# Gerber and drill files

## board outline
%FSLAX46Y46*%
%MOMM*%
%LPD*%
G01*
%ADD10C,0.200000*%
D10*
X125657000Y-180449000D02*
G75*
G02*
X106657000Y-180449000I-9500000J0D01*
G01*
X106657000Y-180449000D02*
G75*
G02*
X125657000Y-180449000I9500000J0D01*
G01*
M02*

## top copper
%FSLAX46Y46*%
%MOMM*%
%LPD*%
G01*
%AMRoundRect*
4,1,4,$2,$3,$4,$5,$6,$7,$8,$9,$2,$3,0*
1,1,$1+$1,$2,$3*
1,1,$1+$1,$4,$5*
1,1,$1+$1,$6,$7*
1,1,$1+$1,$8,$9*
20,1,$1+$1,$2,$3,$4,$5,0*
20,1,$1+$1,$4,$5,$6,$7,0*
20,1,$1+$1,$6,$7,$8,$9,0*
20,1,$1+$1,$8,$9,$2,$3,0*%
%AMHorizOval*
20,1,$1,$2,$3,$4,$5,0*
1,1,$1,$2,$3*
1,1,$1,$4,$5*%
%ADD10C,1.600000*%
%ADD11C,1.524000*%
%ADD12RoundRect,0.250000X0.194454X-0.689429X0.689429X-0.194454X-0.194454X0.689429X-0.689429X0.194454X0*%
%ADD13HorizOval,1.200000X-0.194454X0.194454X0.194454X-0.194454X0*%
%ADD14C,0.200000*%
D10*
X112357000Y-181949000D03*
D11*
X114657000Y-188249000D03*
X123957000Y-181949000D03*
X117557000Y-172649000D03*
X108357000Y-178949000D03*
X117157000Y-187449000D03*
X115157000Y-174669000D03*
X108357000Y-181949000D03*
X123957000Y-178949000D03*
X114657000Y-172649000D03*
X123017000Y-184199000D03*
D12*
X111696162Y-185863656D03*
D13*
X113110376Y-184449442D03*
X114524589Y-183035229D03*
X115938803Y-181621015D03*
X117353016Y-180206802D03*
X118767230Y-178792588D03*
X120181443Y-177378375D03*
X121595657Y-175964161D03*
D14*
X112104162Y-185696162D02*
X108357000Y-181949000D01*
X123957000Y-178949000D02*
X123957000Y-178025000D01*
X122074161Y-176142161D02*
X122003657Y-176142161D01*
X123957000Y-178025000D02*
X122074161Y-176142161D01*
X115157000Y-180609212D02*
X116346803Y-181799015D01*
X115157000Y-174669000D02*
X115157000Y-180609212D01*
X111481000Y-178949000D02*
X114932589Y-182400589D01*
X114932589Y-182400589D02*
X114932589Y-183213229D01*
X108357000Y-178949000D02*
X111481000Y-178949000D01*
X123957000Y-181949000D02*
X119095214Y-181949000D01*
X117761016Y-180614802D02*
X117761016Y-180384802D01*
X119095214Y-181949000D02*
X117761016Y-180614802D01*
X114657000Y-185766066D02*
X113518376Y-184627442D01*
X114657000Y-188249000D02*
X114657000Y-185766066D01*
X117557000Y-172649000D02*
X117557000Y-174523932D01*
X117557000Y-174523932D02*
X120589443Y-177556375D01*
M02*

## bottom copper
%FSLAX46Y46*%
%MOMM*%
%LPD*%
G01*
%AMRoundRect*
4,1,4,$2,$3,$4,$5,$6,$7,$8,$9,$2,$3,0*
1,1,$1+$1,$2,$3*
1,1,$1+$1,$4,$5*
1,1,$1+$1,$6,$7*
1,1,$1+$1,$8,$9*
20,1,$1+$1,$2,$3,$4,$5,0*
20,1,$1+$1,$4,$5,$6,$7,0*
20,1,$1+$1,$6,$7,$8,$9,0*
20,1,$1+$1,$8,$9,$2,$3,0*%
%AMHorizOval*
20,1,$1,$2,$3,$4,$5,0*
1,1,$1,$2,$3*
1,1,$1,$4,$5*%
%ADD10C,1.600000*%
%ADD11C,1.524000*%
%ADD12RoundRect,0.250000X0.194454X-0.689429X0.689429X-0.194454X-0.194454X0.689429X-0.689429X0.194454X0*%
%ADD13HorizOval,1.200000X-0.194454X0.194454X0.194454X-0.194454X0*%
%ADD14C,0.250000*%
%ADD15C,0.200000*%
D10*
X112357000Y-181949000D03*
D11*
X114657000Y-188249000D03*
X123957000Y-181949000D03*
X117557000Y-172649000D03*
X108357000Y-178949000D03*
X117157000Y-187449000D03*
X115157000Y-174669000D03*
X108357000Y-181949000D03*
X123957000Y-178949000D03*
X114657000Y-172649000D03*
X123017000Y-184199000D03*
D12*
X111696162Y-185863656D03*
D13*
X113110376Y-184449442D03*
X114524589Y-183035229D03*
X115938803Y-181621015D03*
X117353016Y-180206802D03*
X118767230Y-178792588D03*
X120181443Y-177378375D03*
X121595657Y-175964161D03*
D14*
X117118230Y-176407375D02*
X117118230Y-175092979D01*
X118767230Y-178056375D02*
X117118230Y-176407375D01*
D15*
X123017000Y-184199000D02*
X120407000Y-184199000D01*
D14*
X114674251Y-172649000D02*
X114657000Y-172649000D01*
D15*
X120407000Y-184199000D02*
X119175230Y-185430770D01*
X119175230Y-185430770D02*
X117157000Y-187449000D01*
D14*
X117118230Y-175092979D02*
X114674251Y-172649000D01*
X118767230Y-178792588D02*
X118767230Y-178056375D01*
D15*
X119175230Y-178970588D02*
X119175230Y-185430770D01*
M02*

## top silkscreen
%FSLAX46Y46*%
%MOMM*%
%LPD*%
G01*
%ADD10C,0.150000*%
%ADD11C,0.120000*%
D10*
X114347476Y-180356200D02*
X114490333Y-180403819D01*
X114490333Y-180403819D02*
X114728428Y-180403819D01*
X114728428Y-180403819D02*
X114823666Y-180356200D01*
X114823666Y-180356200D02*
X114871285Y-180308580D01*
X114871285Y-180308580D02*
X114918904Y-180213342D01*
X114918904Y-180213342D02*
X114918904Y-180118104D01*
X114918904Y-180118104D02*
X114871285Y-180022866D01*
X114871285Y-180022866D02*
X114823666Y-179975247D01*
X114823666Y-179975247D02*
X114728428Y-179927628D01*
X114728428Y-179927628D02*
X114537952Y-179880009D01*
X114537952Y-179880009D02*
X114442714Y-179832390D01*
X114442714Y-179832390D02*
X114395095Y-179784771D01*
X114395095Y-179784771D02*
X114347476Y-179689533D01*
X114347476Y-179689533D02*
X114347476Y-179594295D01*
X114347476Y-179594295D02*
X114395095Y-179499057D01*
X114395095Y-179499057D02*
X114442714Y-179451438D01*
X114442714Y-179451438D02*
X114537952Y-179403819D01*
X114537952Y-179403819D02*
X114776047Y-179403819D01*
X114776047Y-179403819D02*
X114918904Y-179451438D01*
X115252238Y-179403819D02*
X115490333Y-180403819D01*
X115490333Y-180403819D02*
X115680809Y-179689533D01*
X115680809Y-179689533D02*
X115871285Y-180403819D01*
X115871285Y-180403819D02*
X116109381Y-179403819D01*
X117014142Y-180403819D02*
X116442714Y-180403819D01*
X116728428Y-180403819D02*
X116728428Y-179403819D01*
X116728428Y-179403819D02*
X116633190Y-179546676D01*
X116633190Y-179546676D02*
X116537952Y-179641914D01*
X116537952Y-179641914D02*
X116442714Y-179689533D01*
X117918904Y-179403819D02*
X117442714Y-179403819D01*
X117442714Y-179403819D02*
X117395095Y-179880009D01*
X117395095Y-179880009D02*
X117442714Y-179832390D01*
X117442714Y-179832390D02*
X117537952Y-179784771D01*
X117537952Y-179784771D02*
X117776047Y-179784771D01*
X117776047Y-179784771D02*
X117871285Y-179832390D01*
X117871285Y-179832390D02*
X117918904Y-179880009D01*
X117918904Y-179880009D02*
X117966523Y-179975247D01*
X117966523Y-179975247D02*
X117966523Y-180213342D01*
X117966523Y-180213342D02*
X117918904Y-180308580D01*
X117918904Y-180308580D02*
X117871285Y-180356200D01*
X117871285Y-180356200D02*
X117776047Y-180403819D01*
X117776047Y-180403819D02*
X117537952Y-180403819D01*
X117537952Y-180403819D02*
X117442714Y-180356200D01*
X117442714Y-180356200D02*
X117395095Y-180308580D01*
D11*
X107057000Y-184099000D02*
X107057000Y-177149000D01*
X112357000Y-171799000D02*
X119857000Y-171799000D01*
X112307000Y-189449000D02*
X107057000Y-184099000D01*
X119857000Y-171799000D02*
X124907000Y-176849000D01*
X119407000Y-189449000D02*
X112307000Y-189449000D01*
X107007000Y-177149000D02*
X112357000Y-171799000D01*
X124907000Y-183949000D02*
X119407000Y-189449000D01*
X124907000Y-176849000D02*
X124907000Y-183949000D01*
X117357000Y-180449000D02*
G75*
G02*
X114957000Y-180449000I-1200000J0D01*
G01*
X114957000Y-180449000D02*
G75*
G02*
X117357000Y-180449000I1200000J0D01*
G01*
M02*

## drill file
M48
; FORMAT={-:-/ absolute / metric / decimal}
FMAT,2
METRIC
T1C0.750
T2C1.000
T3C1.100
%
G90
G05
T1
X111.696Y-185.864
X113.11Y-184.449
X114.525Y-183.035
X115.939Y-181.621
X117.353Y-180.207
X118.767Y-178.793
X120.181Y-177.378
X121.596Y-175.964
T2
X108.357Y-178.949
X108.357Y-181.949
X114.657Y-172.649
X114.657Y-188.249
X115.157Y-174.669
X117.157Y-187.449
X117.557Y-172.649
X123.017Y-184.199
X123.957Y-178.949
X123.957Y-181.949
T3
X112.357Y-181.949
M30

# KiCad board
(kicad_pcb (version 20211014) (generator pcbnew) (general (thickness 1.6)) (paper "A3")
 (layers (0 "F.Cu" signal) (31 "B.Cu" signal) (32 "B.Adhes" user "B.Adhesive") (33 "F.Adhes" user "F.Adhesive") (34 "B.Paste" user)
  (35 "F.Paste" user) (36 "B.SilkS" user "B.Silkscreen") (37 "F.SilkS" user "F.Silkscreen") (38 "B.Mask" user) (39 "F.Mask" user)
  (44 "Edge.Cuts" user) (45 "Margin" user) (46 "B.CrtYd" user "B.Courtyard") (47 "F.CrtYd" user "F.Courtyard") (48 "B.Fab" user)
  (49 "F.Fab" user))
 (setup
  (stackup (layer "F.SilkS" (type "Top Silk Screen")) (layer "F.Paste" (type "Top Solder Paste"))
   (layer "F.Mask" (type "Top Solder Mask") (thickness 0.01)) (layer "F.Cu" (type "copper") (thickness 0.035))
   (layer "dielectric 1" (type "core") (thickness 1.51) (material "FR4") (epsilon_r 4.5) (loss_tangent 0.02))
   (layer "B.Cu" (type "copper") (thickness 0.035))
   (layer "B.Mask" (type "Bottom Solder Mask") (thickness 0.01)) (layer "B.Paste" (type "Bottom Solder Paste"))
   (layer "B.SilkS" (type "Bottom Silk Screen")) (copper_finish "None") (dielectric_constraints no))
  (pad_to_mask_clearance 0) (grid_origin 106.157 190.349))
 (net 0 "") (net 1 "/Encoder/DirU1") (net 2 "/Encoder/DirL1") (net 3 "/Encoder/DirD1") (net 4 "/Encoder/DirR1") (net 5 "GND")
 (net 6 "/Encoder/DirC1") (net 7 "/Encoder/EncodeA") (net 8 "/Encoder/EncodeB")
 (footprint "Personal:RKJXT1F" (layer "F.Cu") (at 116.157 180.449)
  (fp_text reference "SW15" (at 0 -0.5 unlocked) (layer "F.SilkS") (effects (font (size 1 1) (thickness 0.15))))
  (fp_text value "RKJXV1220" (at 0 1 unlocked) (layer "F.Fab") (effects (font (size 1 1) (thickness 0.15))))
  (fp_line (start -9.1 3.65) (end -9.1 -3.3) (layer "F.SilkS") (width 0.12))
  (fp_line (start -3.8 -8.65) (end 3.7 -8.65) (layer "F.SilkS") (width 0.12))
  (fp_line (start -3.85 9) (end -9.1 3.65) (layer "F.SilkS") (width 0.12))
  (fp_line (start 3.7 -8.65) (end 8.75 -3.6) (layer "F.SilkS") (width 0.12))
  (fp_line (start 3.25 9) (end -3.85 9) (layer "F.SilkS") (width 0.12))
  (fp_line (start -9.15 -3.3) (end -3.8 -8.65) (layer "F.SilkS") (width 0.12))
  (fp_line (start 8.75 3.5) (end 3.25 9) (layer "F.SilkS") (width 0.12))
  (fp_line (start 8.75 -3.6) (end 8.75 3.5) (layer "F.SilkS") (width 0.12))
  (fp_circle (center 0 0) (end 1.2 0) (layer "F.SilkS") (width 0.12) (fill none))
  (pad "" np_thru_hole circle (at -3.8 1.5) (size 1.6 1.6) (drill 1.1) (layers F&B.Cu *.Mask))
  (pad "1" thru_hole circle (at -1.5 7.8) (size 1.524 1.524) (drill 1) (layers F&B.Cu *.Mask) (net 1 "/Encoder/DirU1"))
  (pad "2" thru_hole circle (at 7.8 1.5) (size 1.524 1.524) (drill 1) (layers F&B.Cu *.Mask) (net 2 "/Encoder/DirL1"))
  (pad "3" thru_hole circle (at 1.4 -7.8) (size 1.524 1.524) (drill 1) (layers F&B.Cu *.Mask) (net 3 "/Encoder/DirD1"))
  (pad "4" thru_hole circle (at -7.8 -1.5) (size 1.524 1.524) (drill 1) (layers F&B.Cu *.Mask) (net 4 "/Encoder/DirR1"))
  (pad "5" thru_hole circle (at 1 7) (size 1.524 1.524) (drill 1) (layers F&B.Cu *.Mask) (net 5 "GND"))
  (pad "6" thru_hole circle (at -1 -5.78) (size 1.524 1.524) (drill 1) (layers F&B.Cu *.Mask) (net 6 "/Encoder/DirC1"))
  (pad "A" thru_hole circle (at -7.8 1.5) (size 1.524 1.524) (drill 1) (layers F&B.Cu *.Mask) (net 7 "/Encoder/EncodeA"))
  (pad "B" thru_hole circle (at 7.8 -1.5) (size 1.524 1.524) (drill 1) (layers F&B.Cu *.Mask) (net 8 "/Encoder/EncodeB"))
  (pad "C" thru_hole circle (at -1.5 -7.8) (size 1.524 1.524) (drill 1) (layers F&B.Cu *.Mask) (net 5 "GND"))
  (pad "GND" thru_hole circle (at 6.86 3.75) (size 1.524 1.524) (drill 1) (layers F&B.Cu *.Mask) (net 5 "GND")))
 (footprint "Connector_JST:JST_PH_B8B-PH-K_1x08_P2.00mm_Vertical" (layer "B.Cu") (at 111.696162 185.863656 45)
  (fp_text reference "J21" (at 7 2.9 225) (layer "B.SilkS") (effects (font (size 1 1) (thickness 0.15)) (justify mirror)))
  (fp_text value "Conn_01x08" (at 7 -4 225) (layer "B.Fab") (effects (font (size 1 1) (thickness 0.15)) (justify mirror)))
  (pad "1" thru_hole roundrect (at 0 0 45) (size 1.2 1.75) (drill 0.75) (layers F&B.Cu *.Mask) (roundrect_rratio 0.208333)
   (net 7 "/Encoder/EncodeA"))
  (pad "2" thru_hole oval (at 2 0 45) (size 1.2 1.75) (drill 0.75) (layers F&B.Cu *.Mask) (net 1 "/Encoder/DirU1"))
  (pad "3" thru_hole oval (at 4 0 45) (size 1.2 1.75) (drill 0.75) (layers F&B.Cu *.Mask) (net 4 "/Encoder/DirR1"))
  (pad "4" thru_hole oval (at 6 0 45) (size 1.2 1.75) (drill 0.75) (layers F&B.Cu *.Mask) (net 6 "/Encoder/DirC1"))
  (pad "5" thru_hole oval (at 8 0 45) (size 1.2 1.75) (drill 0.75) (layers F&B.Cu *.Mask) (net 2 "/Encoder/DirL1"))
  (pad "6" thru_hole oval (at 10 0 45) (size 1.2 1.75) (drill 0.75) (layers F&B.Cu *.Mask) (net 5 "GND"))
  (pad "7" thru_hole oval (at 12 0 45) (size 1.2 1.75) (drill 0.75) (layers F&B.Cu *.Mask) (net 3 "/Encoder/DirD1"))
  (pad "8" thru_hole oval (at 14 0 45) (size 1.2 1.75) (drill 0.75) (layers F&B.Cu *.Mask) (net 8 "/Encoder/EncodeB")))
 (gr_circle (center 116.157 180.449) (end 125.657 180.449) (layer "Edge.Cuts") (width 0.2) (fill none))
 (segment (start 117.11823 176.407375) (end 117.11823 175.092979) (width 0.25) (layer "B.Cu") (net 5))
 (segment (start 118.76723 178.056375) (end 117.11823 176.407375) (width 0.25) (layer "B.Cu") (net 5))
 (segment (start 123.017 184.199) (end 120.407 184.199) (width 0.2) (layer "B.Cu") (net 5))
 (segment (start 114.674251 172.649) (end 114.657 172.649) (width 0.25) (layer "B.Cu") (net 5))
 (segment (start 120.407 184.199) (end 119.17523 185.43077) (width 0.2) (layer "B.Cu") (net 5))
 (segment (start 119.17523 185.43077) (end 117.157 187.449) (width 0.2) (layer "B.Cu") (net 5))
 (segment (start 117.11823 175.092979) (end 114.674251 172.649) (width 0.25) (layer "B.Cu") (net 5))
 (segment (start 118.76723 178.792588) (end 118.76723 178.056375) (width 0.25) (layer "B.Cu") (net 5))
 (segment (start 119.17523 178.970588) (end 119.17523 185.43077) (width 0.2) (layer "B.Cu") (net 5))
 (segment (start 112.104162 185.696162) (end 108.357 181.949) (width 0.2) (layer "F.Cu") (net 7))
 (segment (start 123.957 178.949) (end 123.957 178.025) (width 0.2) (layer "F.Cu") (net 8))
 (segment (start 122.074161 176.142161) (end 122.003657 176.142161) (width 0.2) (layer "F.Cu") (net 8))
 (segment (start 123.957 178.025) (end 122.074161 176.142161) (width 0.2) (layer "F.Cu") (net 8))
 (segment (start 115.157 180.609212) (end 116.346803 181.799015) (width 0.2) (layer "F.Cu") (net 6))
 (segment (start 115.157 174.669) (end 115.157 180.609212) (width 0.2) (layer "F.Cu") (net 6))
 (segment (start 111.481 178.949) (end 114.932589 182.400589) (width 0.2) (layer "F.Cu") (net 4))
 (segment (start 114.932589 182.400589) (end 114.932589 183.213229) (width 0.2) (layer "F.Cu") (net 4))
 (segment (start 108.357 178.949) (end 111.481 178.949) (width 0.2) (layer "F.Cu") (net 4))
 (segment (start 123.957 181.949) (end 119.095214 181.949) (width 0.2) (layer "F.Cu") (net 2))
 (segment (start 117.761016 180.614802) (end 117.761016 180.384802) (width 0.2) (layer "F.Cu") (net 2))
 (segment (start 119.095214 181.949) (end 117.761016 180.614802) (width 0.2) (layer "F.Cu") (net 2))
 (segment (start 114.657 185.766066) (end 113.518376 184.627442) (width 0.2) (layer "F.Cu") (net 1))
 (segment (start 114.657 188.249) (end 114.657 185.766066) (width 0.2) (layer "F.Cu") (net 1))
 (segment (start 117.557 172.649) (end 117.557 174.523932) (width 0.2) (layer "F.Cu") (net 3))
 (segment (start 117.557 174.523932) (end 120.589443 177.556375) (width 0.2) (layer "F.Cu") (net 3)))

